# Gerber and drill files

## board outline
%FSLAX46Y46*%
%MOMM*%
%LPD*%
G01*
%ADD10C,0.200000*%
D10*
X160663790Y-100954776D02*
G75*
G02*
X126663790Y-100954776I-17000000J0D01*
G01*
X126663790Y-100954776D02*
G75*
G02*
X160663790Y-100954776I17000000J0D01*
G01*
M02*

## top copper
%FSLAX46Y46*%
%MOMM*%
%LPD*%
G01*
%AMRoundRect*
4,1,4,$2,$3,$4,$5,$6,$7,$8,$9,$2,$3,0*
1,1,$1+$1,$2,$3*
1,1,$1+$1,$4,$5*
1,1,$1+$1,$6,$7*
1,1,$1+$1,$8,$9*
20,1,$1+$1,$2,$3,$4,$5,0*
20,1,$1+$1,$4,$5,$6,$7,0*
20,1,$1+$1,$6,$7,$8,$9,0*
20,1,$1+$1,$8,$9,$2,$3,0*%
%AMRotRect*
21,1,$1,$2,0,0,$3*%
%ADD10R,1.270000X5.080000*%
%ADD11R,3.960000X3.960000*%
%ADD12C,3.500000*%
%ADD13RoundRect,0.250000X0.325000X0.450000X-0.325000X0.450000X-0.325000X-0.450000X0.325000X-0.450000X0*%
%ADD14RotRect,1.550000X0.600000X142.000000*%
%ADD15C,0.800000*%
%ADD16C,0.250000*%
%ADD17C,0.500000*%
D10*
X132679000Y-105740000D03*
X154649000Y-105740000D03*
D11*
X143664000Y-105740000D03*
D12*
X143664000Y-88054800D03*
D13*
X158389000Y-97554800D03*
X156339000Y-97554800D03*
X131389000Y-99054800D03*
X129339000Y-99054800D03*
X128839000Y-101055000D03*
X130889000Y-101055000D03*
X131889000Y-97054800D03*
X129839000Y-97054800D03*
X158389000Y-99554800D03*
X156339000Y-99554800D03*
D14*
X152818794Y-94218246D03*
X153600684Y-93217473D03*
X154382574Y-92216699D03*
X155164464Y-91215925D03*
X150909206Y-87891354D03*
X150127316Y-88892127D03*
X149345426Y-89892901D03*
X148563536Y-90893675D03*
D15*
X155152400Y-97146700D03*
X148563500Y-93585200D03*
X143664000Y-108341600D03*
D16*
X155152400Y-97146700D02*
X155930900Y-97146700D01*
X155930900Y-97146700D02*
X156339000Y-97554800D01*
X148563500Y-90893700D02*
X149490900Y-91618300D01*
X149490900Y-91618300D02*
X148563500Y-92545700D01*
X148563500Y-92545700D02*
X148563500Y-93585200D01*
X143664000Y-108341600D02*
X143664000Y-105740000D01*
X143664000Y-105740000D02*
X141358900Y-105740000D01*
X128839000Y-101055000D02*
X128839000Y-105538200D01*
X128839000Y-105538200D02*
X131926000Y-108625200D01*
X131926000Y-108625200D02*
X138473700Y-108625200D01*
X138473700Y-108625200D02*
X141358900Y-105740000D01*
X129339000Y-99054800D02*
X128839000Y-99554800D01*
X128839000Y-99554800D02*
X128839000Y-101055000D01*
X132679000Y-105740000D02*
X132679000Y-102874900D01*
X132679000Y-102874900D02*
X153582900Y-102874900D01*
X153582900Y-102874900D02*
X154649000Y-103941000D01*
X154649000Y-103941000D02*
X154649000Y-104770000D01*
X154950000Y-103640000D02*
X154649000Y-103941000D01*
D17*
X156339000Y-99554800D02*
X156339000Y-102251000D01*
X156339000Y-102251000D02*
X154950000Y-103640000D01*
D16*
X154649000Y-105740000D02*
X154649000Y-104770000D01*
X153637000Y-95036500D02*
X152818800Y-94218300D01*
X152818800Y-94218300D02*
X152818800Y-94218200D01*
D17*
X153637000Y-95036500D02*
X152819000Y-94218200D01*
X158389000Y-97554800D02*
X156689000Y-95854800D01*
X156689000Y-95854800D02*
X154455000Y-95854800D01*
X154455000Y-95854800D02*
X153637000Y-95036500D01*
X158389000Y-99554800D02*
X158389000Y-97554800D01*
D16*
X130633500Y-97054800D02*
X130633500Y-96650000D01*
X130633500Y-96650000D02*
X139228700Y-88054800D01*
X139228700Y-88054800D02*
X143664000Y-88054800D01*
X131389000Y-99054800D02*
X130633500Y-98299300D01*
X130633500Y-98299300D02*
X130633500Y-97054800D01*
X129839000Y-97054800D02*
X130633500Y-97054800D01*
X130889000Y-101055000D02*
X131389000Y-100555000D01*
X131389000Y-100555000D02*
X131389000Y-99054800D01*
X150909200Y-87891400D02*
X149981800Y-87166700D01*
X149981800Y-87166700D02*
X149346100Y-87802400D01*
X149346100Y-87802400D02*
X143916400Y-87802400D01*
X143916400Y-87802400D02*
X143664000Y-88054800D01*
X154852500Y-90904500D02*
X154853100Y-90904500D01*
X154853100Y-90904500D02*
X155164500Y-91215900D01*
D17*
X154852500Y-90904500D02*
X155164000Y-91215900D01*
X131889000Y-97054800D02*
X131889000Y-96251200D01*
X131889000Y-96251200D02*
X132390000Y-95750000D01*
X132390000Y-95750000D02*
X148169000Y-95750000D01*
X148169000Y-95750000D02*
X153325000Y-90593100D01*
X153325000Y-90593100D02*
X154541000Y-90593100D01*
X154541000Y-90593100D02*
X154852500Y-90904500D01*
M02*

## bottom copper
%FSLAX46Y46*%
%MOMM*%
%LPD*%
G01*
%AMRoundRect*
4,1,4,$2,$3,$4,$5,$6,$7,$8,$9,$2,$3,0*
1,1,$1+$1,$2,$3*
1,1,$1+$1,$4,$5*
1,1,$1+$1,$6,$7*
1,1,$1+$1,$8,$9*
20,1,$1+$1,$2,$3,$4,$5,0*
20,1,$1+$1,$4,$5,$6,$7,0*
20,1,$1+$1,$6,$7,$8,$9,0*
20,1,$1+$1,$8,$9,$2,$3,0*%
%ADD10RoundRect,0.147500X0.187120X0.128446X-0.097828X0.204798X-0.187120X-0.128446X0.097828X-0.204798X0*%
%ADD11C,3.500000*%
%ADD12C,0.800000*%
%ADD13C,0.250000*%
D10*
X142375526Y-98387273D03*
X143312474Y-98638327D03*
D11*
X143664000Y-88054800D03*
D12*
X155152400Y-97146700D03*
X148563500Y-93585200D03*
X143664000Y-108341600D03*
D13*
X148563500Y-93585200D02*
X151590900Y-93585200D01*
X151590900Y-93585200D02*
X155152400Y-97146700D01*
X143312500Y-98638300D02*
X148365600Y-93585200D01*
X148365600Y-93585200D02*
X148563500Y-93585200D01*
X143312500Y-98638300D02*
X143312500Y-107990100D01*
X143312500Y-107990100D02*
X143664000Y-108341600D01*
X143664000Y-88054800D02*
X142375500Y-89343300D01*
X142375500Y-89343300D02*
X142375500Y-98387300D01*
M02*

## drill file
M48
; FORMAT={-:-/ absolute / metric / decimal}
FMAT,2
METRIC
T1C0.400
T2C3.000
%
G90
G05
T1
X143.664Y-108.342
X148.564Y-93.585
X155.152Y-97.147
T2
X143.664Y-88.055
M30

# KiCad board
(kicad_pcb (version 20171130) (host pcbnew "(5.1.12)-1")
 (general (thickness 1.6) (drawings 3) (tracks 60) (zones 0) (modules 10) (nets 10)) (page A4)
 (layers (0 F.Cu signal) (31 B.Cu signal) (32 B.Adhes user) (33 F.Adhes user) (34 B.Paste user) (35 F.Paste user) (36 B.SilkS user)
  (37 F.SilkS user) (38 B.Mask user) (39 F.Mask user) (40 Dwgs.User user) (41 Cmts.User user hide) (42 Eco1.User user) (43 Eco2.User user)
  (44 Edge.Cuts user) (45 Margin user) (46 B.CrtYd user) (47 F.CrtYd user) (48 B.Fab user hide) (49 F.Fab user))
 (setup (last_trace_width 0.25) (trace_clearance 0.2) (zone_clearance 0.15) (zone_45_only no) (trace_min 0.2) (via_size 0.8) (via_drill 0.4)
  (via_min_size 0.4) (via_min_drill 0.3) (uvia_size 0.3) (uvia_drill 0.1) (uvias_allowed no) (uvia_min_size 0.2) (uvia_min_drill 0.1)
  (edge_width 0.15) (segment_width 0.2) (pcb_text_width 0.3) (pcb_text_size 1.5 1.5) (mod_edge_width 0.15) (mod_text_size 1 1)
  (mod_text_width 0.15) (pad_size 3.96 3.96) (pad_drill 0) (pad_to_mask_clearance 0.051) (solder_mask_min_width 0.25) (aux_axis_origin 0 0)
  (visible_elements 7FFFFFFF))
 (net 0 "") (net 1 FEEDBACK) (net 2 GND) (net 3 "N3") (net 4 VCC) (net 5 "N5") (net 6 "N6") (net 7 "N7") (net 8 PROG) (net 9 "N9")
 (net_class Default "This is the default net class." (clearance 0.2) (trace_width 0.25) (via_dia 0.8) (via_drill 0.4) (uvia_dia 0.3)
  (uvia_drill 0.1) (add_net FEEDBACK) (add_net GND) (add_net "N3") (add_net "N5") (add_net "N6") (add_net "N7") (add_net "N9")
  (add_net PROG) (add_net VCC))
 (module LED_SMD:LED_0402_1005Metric (layer B.Cu) (at 142.844 98.5128 165)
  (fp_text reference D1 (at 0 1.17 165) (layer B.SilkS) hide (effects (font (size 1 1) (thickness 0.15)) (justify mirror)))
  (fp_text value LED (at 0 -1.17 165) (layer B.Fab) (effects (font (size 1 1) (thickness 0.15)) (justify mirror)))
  (pad 2 smd roundrect (at 0.485 0 165) (size 0.59 0.64) (layers B.Cu B.Paste B.Mask) (roundrect_rratio 0.25) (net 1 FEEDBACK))
  (pad 1 smd roundrect (at -0.485 0 165) (size 0.59 0.64) (layers B.Cu B.Paste B.Mask) (roundrect_rratio 0.25) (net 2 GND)))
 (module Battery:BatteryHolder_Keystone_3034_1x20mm (layer F.Cu) (at 143.664 105.74)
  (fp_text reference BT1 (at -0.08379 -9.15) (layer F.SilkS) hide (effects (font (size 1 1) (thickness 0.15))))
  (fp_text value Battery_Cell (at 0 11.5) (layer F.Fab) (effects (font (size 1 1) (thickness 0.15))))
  (pad 1 smd rect (at -10.985 0) (size 1.27 5.08) (layers F.Cu F.Paste F.Mask) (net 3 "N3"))
  (pad 1 smd rect (at 10.985 0) (size 1.27 5.08) (layers F.Cu F.Paste F.Mask) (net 3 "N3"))
  (pad 2 smd rect (at 0 0) (size 3.96 3.96) (layers F.Cu F.Paste F.Mask) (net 2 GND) (zone_connect 2)))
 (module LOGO (layer B.Cu) (at 144.12 102.37 180)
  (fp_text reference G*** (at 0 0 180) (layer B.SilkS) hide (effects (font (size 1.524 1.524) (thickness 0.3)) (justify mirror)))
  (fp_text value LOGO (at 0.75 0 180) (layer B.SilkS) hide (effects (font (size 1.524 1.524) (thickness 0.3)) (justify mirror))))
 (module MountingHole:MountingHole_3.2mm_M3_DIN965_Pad (layer B.Cu) (at 143.664 88.0548 180)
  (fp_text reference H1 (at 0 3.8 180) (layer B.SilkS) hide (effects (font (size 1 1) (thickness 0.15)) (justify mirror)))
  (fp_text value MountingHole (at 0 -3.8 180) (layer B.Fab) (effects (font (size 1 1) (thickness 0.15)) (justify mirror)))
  (pad 1 thru_hole circle (at 0 0 180) (size 3.5 3.5) (drill 3) (layers *.Cu *.Mask) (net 1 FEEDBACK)))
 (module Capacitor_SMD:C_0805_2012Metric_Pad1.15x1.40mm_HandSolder (layer F.Cu) (at 157.364 97.5548 180)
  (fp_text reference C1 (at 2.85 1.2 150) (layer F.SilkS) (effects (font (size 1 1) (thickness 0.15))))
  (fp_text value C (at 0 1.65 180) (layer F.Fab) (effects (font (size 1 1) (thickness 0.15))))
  (pad 1 smd roundrect (at -1.025 0 180) (size 1.15 1.4) (layers F.Cu F.Paste F.Mask) (roundrect_rratio 0.217391) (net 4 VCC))
  (pad 2 smd roundrect (at 1.025 0 180) (size 1.15 1.4) (layers F.Cu F.Paste F.Mask) (roundrect_rratio 0.217391) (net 2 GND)))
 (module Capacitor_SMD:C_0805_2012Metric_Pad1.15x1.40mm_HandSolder (layer F.Cu) (at 130.364 99.0548 180)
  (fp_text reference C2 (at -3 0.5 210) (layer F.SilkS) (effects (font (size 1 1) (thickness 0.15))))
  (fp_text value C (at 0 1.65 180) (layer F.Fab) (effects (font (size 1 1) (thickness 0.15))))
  (pad 1 smd roundrect (at -1.025 0 180) (size 1.15 1.4) (layers F.Cu F.Paste F.Mask) (roundrect_rratio 0.217391) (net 1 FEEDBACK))
  (pad 2 smd roundrect (at 1.025 0 180) (size 1.15 1.4) (layers F.Cu F.Paste F.Mask) (roundrect_rratio 0.217391) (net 2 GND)))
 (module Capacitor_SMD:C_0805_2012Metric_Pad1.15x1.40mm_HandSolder (layer F.Cu) (at 129.864 101.055 180)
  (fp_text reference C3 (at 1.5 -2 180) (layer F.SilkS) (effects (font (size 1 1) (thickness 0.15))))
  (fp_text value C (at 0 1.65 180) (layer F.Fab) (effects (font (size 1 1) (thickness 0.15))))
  (pad 2 smd roundrect (at 1.025 0 180) (size 1.15 1.4) (layers F.Cu F.Paste F.Mask) (roundrect_rratio 0.217391) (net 2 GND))
  (pad 1 smd roundrect (at -1.025 0 180) (size 1.15 1.4) (layers F.Cu F.Paste F.Mask) (roundrect_rratio 0.217391) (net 1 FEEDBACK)))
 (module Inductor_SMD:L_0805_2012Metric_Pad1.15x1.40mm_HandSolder (layer F.Cu) (at 130.864 97.0548 180)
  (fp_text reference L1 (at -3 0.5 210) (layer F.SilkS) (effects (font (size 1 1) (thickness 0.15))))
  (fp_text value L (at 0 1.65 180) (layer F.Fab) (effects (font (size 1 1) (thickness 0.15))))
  (pad 1 smd roundrect (at -1.025 0 180) (size 1.15 1.4) (layers F.Cu F.Paste F.Mask) (roundrect_rratio 0.217391) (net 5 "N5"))
  (pad 2 smd roundrect (at 1.025 0 180) (size 1.15 1.4) (layers F.Cu F.Paste F.Mask) (roundrect_rratio 0.217391) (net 1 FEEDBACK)))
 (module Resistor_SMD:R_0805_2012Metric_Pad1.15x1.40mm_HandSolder (layer F.Cu) (at 157.364 99.5548 180)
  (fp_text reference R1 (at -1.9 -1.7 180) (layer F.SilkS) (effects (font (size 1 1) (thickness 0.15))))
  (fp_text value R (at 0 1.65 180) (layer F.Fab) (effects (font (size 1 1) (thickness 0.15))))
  (pad 1 smd roundrect (at -1.025 0 180) (size 1.15 1.4) (layers F.Cu F.Paste F.Mask) (roundrect_rratio 0.217391) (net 4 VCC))
  (pad 2 smd roundrect (at 1.025 0 180) (size 1.15 1.4) (layers F.Cu F.Paste F.Mask) (roundrect_rratio 0.217391) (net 3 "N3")))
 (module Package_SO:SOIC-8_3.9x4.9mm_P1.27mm (layer F.Cu) (at 151.864 91.0548 142)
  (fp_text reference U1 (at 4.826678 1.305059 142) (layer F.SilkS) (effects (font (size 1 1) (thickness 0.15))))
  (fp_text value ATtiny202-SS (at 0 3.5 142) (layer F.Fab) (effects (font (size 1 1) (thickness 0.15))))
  (pad 1 smd rect (at -2.7 -1.905 142) (size 1.55 0.6) (layers F.Cu F.Paste F.Mask) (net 4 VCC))
  (pad 2 smd rect (at -2.7 -0.635 142) (size 1.55 0.6) (layers F.Cu F.Paste F.Mask) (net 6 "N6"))
  (pad 3 smd rect (at -2.7 0.635 142) (size 1.55 0.6) (layers F.Cu F.Paste F.Mask) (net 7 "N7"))
  (pad 4 smd rect (at -2.7 1.905 142) (size 1.55 0.6) (layers F.Cu F.Paste F.Mask) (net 5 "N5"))
  (pad 5 smd rect (at 2.7 1.905 142) (size 1.55 0.6) (layers F.Cu F.Paste F.Mask) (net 1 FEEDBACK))
  (pad 6 smd rect (at 2.7 0.635 142) (size 1.55 0.6) (layers F.Cu F.Paste F.Mask) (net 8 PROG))
  (pad 7 smd rect (at 2.7 -0.635 142) (size 1.55 0.6) (layers F.Cu F.Paste F.Mask) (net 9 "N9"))
  (pad 8 smd rect (at 2.7 -1.905 142) (size 1.55 0.6) (layers F.Cu F.Paste F.Mask) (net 2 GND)))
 (gr_circle (center 143.66379 100.954776) (end 126.66379 100.954776) (layer Edge.Cuts) (width 0.2))
 (segment (start 155.1524 97.1467) (end 155.9309 97.1467) (width 0.25) (layer F.Cu) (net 2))
 (segment (start 155.9309 97.1467) (end 156.339 97.5548) (width 0.25) (layer F.Cu) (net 2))
 (segment (start 148.5635 93.5852) (end 151.5909 93.5852) (width 0.25) (layer B.Cu) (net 2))
 (segment (start 151.5909 93.5852) (end 155.1524 97.1467) (width 0.25) (layer B.Cu) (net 2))
 (segment (start 143.3125 98.6383) (end 148.3656 93.5852) (width 0.25) (layer B.Cu) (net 2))
 (segment (start 148.3656 93.5852) (end 148.5635 93.5852) (width 0.25) (layer B.Cu) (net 2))
 (segment (start 148.5635 90.8937) (end 149.4909 91.6183) (width 0.25) (layer F.Cu) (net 2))
 (segment (start 149.4909 91.6183) (end 148.5635 92.5457) (width 0.25) (layer F.Cu) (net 2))
 (segment (start 148.5635 92.5457) (end 148.5635 93.5852) (width 0.25) (layer F.Cu) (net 2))
 (segment (start 143.664 108.3416) (end 143.664 105.74) (width 0.25) (layer F.Cu) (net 2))
 (segment (start 143.3125 98.6383) (end 143.3125 107.9901) (width 0.25) (layer B.Cu) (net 2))
 (segment (start 143.3125 107.9901) (end 143.664 108.3416) (width 0.25) (layer B.Cu) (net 2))
 (segment (start 143.664 105.74) (end 141.3589 105.74) (width 0.25) (layer F.Cu) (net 2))
 (segment (start 128.839 101.055) (end 128.839 105.5382) (width 0.25) (layer F.Cu) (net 2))
 (segment (start 128.839 105.5382) (end 131.926 108.6252) (width 0.25) (layer F.Cu) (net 2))
 (segment (start 131.926 108.6252) (end 138.4737 108.6252) (width 0.25) (layer F.Cu) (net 2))
 (segment (start 138.4737 108.6252) (end 141.3589 105.74) (width 0.25) (layer F.Cu) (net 2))
 (segment (start 129.339 99.0548) (end 128.839 99.5548) (width 0.25) (layer F.Cu) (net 2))
 (segment (start 128.839 99.5548) (end 128.839 101.055) (width 0.25) (layer F.Cu) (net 2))
 (via (at 155.1524 97.1467) (size 0.8) (layers F.Cu B.Cu) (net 2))
 (via (at 148.5635 93.5852) (size 0.8) (layers F.Cu B.Cu) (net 2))
 (via (at 143.664 108.3416) (size 0.8) (layers F.Cu B.Cu) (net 2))
 (segment (start 132.679 105.74) (end 132.679 102.8749) (width 0.25) (layer F.Cu) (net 3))
 (segment (start 132.679 102.8749) (end 153.5829 102.8749) (width 0.25) (layer F.Cu) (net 3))
 (segment (start 153.5829 102.8749) (end 154.649 103.941) (width 0.25) (layer F.Cu) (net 3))
 (segment (start 154.649 103.941) (end 154.649 104.77) (width 0.25) (layer F.Cu) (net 3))
 (segment (start 154.95 103.64) (end 154.649 103.941) (width 0.25) (layer F.Cu) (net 3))
 (segment (start 156.339 99.5548) (end 156.339 102.251) (width 0.5) (layer F.Cu) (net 3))
 (segment (start 156.339 102.251) (end 154.95 103.64) (width 0.5) (layer F.Cu) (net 3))
 (segment (start 154.649 105.74) (end 154.649 104.77) (width 0.25) (layer F.Cu) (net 3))
 (segment (start 153.637 95.0365) (end 152.8188 94.2183) (width 0.25) (layer F.Cu) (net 4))
 (segment (start 152.8188 94.2183) (end 152.8188 94.2182) (width 0.25) (layer F.Cu) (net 4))
 (segment (start 153.637 95.0365) (end 152.819 94.2182) (width 0.5) (layer F.Cu) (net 4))
 (segment (start 158.389 97.5548) (end 156.689 95.8548) (width 0.5) (layer F.Cu) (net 4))
 (segment (start 156.689 95.8548) (end 154.455 95.8548) (width 0.5) (layer F.Cu) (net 4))
 (segment (start 154.455 95.8548) (end 153.637 95.0365) (width 0.5) (layer F.Cu) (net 4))
 (segment (start 158.389 99.5548) (end 158.389 97.5548) (width 0.5) (layer F.Cu) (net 4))
 (segment (start 143.664 88.0548) (end 142.3755 89.3433) (width 0.25) (layer B.Cu) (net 1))
 (segment (start 142.3755 89.3433) (end 142.3755 98.3873) (width 0.25) (layer B.Cu) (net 1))
 (segment (start 130.6335 97.0548) (end 130.6335 96.65) (width 0.25) (layer F.Cu) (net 1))
 (segment (start 130.6335 96.65) (end 139.2287 88.0548) (width 0.25) (layer F.Cu) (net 1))
 (segment (start 139.2287 88.0548) (end 143.664 88.0548) (width 0.25) (layer F.Cu) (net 1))
 (segment (start 131.389 99.0548) (end 130.6335 98.2993) (width 0.25) (layer F.Cu) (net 1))
 (segment (start 130.6335 98.2993) (end 130.6335 97.0548) (width 0.25) (layer F.Cu) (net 1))
 (segment (start 129.839 97.0548) (end 130.6335 97.0548) (width 0.25) (layer F.Cu) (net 1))
 (segment (start 130.889 101.055) (end 131.389 100.555) (width 0.25) (layer F.Cu) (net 1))
 (segment (start 131.389 100.555) (end 131.389 99.0548) (width 0.25) (layer F.Cu) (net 1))
 (segment (start 150.9092 87.8914) (end 149.9818 87.1667) (width 0.25) (layer F.Cu) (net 1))
 (segment (start 149.9818 87.1667) (end 149.3461 87.8024) (width 0.25) (layer F.Cu) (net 1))
 (segment (start 149.3461 87.8024) (end 143.9164 87.8024) (width 0.25) (layer F.Cu) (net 1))
 (segment (start 143.9164 87.8024) (end 143.664 88.0548) (width 0.25) (layer F.Cu) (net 1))
 (segment (start 154.8525 90.9045) (end 154.8531 90.9045) (width 0.25) (layer F.Cu) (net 5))
 (segment (start 154.8531 90.9045) (end 155.1645 91.2159) (width 0.25) (layer F.Cu) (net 5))
 (segment (start 154.8525 90.9045) (end 155.164 91.2159) (width 0.5) (layer F.Cu) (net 5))
 (segment (start 131.889 97.0548) (end 131.889 96.2512) (width 0.5) (layer F.Cu) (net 5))
 (segment (start 131.889 96.2512) (end 132.39 95.75) (width 0.5) (layer F.Cu) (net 5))
 (segment (start 132.39 95.75) (end 148.169 95.75) (width 0.5) (layer F.Cu) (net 5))
 (segment (start 148.169 95.75) (end 153.325 90.5931) (width 0.5) (layer F.Cu) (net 5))
 (segment (start 153.325 90.5931) (end 154.541 90.5931) (width 0.5) (layer F.Cu) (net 5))
 (segment (start 154.541 90.5931) (end 154.8525 90.9045) (width 0.5) (layer F.Cu) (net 5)))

